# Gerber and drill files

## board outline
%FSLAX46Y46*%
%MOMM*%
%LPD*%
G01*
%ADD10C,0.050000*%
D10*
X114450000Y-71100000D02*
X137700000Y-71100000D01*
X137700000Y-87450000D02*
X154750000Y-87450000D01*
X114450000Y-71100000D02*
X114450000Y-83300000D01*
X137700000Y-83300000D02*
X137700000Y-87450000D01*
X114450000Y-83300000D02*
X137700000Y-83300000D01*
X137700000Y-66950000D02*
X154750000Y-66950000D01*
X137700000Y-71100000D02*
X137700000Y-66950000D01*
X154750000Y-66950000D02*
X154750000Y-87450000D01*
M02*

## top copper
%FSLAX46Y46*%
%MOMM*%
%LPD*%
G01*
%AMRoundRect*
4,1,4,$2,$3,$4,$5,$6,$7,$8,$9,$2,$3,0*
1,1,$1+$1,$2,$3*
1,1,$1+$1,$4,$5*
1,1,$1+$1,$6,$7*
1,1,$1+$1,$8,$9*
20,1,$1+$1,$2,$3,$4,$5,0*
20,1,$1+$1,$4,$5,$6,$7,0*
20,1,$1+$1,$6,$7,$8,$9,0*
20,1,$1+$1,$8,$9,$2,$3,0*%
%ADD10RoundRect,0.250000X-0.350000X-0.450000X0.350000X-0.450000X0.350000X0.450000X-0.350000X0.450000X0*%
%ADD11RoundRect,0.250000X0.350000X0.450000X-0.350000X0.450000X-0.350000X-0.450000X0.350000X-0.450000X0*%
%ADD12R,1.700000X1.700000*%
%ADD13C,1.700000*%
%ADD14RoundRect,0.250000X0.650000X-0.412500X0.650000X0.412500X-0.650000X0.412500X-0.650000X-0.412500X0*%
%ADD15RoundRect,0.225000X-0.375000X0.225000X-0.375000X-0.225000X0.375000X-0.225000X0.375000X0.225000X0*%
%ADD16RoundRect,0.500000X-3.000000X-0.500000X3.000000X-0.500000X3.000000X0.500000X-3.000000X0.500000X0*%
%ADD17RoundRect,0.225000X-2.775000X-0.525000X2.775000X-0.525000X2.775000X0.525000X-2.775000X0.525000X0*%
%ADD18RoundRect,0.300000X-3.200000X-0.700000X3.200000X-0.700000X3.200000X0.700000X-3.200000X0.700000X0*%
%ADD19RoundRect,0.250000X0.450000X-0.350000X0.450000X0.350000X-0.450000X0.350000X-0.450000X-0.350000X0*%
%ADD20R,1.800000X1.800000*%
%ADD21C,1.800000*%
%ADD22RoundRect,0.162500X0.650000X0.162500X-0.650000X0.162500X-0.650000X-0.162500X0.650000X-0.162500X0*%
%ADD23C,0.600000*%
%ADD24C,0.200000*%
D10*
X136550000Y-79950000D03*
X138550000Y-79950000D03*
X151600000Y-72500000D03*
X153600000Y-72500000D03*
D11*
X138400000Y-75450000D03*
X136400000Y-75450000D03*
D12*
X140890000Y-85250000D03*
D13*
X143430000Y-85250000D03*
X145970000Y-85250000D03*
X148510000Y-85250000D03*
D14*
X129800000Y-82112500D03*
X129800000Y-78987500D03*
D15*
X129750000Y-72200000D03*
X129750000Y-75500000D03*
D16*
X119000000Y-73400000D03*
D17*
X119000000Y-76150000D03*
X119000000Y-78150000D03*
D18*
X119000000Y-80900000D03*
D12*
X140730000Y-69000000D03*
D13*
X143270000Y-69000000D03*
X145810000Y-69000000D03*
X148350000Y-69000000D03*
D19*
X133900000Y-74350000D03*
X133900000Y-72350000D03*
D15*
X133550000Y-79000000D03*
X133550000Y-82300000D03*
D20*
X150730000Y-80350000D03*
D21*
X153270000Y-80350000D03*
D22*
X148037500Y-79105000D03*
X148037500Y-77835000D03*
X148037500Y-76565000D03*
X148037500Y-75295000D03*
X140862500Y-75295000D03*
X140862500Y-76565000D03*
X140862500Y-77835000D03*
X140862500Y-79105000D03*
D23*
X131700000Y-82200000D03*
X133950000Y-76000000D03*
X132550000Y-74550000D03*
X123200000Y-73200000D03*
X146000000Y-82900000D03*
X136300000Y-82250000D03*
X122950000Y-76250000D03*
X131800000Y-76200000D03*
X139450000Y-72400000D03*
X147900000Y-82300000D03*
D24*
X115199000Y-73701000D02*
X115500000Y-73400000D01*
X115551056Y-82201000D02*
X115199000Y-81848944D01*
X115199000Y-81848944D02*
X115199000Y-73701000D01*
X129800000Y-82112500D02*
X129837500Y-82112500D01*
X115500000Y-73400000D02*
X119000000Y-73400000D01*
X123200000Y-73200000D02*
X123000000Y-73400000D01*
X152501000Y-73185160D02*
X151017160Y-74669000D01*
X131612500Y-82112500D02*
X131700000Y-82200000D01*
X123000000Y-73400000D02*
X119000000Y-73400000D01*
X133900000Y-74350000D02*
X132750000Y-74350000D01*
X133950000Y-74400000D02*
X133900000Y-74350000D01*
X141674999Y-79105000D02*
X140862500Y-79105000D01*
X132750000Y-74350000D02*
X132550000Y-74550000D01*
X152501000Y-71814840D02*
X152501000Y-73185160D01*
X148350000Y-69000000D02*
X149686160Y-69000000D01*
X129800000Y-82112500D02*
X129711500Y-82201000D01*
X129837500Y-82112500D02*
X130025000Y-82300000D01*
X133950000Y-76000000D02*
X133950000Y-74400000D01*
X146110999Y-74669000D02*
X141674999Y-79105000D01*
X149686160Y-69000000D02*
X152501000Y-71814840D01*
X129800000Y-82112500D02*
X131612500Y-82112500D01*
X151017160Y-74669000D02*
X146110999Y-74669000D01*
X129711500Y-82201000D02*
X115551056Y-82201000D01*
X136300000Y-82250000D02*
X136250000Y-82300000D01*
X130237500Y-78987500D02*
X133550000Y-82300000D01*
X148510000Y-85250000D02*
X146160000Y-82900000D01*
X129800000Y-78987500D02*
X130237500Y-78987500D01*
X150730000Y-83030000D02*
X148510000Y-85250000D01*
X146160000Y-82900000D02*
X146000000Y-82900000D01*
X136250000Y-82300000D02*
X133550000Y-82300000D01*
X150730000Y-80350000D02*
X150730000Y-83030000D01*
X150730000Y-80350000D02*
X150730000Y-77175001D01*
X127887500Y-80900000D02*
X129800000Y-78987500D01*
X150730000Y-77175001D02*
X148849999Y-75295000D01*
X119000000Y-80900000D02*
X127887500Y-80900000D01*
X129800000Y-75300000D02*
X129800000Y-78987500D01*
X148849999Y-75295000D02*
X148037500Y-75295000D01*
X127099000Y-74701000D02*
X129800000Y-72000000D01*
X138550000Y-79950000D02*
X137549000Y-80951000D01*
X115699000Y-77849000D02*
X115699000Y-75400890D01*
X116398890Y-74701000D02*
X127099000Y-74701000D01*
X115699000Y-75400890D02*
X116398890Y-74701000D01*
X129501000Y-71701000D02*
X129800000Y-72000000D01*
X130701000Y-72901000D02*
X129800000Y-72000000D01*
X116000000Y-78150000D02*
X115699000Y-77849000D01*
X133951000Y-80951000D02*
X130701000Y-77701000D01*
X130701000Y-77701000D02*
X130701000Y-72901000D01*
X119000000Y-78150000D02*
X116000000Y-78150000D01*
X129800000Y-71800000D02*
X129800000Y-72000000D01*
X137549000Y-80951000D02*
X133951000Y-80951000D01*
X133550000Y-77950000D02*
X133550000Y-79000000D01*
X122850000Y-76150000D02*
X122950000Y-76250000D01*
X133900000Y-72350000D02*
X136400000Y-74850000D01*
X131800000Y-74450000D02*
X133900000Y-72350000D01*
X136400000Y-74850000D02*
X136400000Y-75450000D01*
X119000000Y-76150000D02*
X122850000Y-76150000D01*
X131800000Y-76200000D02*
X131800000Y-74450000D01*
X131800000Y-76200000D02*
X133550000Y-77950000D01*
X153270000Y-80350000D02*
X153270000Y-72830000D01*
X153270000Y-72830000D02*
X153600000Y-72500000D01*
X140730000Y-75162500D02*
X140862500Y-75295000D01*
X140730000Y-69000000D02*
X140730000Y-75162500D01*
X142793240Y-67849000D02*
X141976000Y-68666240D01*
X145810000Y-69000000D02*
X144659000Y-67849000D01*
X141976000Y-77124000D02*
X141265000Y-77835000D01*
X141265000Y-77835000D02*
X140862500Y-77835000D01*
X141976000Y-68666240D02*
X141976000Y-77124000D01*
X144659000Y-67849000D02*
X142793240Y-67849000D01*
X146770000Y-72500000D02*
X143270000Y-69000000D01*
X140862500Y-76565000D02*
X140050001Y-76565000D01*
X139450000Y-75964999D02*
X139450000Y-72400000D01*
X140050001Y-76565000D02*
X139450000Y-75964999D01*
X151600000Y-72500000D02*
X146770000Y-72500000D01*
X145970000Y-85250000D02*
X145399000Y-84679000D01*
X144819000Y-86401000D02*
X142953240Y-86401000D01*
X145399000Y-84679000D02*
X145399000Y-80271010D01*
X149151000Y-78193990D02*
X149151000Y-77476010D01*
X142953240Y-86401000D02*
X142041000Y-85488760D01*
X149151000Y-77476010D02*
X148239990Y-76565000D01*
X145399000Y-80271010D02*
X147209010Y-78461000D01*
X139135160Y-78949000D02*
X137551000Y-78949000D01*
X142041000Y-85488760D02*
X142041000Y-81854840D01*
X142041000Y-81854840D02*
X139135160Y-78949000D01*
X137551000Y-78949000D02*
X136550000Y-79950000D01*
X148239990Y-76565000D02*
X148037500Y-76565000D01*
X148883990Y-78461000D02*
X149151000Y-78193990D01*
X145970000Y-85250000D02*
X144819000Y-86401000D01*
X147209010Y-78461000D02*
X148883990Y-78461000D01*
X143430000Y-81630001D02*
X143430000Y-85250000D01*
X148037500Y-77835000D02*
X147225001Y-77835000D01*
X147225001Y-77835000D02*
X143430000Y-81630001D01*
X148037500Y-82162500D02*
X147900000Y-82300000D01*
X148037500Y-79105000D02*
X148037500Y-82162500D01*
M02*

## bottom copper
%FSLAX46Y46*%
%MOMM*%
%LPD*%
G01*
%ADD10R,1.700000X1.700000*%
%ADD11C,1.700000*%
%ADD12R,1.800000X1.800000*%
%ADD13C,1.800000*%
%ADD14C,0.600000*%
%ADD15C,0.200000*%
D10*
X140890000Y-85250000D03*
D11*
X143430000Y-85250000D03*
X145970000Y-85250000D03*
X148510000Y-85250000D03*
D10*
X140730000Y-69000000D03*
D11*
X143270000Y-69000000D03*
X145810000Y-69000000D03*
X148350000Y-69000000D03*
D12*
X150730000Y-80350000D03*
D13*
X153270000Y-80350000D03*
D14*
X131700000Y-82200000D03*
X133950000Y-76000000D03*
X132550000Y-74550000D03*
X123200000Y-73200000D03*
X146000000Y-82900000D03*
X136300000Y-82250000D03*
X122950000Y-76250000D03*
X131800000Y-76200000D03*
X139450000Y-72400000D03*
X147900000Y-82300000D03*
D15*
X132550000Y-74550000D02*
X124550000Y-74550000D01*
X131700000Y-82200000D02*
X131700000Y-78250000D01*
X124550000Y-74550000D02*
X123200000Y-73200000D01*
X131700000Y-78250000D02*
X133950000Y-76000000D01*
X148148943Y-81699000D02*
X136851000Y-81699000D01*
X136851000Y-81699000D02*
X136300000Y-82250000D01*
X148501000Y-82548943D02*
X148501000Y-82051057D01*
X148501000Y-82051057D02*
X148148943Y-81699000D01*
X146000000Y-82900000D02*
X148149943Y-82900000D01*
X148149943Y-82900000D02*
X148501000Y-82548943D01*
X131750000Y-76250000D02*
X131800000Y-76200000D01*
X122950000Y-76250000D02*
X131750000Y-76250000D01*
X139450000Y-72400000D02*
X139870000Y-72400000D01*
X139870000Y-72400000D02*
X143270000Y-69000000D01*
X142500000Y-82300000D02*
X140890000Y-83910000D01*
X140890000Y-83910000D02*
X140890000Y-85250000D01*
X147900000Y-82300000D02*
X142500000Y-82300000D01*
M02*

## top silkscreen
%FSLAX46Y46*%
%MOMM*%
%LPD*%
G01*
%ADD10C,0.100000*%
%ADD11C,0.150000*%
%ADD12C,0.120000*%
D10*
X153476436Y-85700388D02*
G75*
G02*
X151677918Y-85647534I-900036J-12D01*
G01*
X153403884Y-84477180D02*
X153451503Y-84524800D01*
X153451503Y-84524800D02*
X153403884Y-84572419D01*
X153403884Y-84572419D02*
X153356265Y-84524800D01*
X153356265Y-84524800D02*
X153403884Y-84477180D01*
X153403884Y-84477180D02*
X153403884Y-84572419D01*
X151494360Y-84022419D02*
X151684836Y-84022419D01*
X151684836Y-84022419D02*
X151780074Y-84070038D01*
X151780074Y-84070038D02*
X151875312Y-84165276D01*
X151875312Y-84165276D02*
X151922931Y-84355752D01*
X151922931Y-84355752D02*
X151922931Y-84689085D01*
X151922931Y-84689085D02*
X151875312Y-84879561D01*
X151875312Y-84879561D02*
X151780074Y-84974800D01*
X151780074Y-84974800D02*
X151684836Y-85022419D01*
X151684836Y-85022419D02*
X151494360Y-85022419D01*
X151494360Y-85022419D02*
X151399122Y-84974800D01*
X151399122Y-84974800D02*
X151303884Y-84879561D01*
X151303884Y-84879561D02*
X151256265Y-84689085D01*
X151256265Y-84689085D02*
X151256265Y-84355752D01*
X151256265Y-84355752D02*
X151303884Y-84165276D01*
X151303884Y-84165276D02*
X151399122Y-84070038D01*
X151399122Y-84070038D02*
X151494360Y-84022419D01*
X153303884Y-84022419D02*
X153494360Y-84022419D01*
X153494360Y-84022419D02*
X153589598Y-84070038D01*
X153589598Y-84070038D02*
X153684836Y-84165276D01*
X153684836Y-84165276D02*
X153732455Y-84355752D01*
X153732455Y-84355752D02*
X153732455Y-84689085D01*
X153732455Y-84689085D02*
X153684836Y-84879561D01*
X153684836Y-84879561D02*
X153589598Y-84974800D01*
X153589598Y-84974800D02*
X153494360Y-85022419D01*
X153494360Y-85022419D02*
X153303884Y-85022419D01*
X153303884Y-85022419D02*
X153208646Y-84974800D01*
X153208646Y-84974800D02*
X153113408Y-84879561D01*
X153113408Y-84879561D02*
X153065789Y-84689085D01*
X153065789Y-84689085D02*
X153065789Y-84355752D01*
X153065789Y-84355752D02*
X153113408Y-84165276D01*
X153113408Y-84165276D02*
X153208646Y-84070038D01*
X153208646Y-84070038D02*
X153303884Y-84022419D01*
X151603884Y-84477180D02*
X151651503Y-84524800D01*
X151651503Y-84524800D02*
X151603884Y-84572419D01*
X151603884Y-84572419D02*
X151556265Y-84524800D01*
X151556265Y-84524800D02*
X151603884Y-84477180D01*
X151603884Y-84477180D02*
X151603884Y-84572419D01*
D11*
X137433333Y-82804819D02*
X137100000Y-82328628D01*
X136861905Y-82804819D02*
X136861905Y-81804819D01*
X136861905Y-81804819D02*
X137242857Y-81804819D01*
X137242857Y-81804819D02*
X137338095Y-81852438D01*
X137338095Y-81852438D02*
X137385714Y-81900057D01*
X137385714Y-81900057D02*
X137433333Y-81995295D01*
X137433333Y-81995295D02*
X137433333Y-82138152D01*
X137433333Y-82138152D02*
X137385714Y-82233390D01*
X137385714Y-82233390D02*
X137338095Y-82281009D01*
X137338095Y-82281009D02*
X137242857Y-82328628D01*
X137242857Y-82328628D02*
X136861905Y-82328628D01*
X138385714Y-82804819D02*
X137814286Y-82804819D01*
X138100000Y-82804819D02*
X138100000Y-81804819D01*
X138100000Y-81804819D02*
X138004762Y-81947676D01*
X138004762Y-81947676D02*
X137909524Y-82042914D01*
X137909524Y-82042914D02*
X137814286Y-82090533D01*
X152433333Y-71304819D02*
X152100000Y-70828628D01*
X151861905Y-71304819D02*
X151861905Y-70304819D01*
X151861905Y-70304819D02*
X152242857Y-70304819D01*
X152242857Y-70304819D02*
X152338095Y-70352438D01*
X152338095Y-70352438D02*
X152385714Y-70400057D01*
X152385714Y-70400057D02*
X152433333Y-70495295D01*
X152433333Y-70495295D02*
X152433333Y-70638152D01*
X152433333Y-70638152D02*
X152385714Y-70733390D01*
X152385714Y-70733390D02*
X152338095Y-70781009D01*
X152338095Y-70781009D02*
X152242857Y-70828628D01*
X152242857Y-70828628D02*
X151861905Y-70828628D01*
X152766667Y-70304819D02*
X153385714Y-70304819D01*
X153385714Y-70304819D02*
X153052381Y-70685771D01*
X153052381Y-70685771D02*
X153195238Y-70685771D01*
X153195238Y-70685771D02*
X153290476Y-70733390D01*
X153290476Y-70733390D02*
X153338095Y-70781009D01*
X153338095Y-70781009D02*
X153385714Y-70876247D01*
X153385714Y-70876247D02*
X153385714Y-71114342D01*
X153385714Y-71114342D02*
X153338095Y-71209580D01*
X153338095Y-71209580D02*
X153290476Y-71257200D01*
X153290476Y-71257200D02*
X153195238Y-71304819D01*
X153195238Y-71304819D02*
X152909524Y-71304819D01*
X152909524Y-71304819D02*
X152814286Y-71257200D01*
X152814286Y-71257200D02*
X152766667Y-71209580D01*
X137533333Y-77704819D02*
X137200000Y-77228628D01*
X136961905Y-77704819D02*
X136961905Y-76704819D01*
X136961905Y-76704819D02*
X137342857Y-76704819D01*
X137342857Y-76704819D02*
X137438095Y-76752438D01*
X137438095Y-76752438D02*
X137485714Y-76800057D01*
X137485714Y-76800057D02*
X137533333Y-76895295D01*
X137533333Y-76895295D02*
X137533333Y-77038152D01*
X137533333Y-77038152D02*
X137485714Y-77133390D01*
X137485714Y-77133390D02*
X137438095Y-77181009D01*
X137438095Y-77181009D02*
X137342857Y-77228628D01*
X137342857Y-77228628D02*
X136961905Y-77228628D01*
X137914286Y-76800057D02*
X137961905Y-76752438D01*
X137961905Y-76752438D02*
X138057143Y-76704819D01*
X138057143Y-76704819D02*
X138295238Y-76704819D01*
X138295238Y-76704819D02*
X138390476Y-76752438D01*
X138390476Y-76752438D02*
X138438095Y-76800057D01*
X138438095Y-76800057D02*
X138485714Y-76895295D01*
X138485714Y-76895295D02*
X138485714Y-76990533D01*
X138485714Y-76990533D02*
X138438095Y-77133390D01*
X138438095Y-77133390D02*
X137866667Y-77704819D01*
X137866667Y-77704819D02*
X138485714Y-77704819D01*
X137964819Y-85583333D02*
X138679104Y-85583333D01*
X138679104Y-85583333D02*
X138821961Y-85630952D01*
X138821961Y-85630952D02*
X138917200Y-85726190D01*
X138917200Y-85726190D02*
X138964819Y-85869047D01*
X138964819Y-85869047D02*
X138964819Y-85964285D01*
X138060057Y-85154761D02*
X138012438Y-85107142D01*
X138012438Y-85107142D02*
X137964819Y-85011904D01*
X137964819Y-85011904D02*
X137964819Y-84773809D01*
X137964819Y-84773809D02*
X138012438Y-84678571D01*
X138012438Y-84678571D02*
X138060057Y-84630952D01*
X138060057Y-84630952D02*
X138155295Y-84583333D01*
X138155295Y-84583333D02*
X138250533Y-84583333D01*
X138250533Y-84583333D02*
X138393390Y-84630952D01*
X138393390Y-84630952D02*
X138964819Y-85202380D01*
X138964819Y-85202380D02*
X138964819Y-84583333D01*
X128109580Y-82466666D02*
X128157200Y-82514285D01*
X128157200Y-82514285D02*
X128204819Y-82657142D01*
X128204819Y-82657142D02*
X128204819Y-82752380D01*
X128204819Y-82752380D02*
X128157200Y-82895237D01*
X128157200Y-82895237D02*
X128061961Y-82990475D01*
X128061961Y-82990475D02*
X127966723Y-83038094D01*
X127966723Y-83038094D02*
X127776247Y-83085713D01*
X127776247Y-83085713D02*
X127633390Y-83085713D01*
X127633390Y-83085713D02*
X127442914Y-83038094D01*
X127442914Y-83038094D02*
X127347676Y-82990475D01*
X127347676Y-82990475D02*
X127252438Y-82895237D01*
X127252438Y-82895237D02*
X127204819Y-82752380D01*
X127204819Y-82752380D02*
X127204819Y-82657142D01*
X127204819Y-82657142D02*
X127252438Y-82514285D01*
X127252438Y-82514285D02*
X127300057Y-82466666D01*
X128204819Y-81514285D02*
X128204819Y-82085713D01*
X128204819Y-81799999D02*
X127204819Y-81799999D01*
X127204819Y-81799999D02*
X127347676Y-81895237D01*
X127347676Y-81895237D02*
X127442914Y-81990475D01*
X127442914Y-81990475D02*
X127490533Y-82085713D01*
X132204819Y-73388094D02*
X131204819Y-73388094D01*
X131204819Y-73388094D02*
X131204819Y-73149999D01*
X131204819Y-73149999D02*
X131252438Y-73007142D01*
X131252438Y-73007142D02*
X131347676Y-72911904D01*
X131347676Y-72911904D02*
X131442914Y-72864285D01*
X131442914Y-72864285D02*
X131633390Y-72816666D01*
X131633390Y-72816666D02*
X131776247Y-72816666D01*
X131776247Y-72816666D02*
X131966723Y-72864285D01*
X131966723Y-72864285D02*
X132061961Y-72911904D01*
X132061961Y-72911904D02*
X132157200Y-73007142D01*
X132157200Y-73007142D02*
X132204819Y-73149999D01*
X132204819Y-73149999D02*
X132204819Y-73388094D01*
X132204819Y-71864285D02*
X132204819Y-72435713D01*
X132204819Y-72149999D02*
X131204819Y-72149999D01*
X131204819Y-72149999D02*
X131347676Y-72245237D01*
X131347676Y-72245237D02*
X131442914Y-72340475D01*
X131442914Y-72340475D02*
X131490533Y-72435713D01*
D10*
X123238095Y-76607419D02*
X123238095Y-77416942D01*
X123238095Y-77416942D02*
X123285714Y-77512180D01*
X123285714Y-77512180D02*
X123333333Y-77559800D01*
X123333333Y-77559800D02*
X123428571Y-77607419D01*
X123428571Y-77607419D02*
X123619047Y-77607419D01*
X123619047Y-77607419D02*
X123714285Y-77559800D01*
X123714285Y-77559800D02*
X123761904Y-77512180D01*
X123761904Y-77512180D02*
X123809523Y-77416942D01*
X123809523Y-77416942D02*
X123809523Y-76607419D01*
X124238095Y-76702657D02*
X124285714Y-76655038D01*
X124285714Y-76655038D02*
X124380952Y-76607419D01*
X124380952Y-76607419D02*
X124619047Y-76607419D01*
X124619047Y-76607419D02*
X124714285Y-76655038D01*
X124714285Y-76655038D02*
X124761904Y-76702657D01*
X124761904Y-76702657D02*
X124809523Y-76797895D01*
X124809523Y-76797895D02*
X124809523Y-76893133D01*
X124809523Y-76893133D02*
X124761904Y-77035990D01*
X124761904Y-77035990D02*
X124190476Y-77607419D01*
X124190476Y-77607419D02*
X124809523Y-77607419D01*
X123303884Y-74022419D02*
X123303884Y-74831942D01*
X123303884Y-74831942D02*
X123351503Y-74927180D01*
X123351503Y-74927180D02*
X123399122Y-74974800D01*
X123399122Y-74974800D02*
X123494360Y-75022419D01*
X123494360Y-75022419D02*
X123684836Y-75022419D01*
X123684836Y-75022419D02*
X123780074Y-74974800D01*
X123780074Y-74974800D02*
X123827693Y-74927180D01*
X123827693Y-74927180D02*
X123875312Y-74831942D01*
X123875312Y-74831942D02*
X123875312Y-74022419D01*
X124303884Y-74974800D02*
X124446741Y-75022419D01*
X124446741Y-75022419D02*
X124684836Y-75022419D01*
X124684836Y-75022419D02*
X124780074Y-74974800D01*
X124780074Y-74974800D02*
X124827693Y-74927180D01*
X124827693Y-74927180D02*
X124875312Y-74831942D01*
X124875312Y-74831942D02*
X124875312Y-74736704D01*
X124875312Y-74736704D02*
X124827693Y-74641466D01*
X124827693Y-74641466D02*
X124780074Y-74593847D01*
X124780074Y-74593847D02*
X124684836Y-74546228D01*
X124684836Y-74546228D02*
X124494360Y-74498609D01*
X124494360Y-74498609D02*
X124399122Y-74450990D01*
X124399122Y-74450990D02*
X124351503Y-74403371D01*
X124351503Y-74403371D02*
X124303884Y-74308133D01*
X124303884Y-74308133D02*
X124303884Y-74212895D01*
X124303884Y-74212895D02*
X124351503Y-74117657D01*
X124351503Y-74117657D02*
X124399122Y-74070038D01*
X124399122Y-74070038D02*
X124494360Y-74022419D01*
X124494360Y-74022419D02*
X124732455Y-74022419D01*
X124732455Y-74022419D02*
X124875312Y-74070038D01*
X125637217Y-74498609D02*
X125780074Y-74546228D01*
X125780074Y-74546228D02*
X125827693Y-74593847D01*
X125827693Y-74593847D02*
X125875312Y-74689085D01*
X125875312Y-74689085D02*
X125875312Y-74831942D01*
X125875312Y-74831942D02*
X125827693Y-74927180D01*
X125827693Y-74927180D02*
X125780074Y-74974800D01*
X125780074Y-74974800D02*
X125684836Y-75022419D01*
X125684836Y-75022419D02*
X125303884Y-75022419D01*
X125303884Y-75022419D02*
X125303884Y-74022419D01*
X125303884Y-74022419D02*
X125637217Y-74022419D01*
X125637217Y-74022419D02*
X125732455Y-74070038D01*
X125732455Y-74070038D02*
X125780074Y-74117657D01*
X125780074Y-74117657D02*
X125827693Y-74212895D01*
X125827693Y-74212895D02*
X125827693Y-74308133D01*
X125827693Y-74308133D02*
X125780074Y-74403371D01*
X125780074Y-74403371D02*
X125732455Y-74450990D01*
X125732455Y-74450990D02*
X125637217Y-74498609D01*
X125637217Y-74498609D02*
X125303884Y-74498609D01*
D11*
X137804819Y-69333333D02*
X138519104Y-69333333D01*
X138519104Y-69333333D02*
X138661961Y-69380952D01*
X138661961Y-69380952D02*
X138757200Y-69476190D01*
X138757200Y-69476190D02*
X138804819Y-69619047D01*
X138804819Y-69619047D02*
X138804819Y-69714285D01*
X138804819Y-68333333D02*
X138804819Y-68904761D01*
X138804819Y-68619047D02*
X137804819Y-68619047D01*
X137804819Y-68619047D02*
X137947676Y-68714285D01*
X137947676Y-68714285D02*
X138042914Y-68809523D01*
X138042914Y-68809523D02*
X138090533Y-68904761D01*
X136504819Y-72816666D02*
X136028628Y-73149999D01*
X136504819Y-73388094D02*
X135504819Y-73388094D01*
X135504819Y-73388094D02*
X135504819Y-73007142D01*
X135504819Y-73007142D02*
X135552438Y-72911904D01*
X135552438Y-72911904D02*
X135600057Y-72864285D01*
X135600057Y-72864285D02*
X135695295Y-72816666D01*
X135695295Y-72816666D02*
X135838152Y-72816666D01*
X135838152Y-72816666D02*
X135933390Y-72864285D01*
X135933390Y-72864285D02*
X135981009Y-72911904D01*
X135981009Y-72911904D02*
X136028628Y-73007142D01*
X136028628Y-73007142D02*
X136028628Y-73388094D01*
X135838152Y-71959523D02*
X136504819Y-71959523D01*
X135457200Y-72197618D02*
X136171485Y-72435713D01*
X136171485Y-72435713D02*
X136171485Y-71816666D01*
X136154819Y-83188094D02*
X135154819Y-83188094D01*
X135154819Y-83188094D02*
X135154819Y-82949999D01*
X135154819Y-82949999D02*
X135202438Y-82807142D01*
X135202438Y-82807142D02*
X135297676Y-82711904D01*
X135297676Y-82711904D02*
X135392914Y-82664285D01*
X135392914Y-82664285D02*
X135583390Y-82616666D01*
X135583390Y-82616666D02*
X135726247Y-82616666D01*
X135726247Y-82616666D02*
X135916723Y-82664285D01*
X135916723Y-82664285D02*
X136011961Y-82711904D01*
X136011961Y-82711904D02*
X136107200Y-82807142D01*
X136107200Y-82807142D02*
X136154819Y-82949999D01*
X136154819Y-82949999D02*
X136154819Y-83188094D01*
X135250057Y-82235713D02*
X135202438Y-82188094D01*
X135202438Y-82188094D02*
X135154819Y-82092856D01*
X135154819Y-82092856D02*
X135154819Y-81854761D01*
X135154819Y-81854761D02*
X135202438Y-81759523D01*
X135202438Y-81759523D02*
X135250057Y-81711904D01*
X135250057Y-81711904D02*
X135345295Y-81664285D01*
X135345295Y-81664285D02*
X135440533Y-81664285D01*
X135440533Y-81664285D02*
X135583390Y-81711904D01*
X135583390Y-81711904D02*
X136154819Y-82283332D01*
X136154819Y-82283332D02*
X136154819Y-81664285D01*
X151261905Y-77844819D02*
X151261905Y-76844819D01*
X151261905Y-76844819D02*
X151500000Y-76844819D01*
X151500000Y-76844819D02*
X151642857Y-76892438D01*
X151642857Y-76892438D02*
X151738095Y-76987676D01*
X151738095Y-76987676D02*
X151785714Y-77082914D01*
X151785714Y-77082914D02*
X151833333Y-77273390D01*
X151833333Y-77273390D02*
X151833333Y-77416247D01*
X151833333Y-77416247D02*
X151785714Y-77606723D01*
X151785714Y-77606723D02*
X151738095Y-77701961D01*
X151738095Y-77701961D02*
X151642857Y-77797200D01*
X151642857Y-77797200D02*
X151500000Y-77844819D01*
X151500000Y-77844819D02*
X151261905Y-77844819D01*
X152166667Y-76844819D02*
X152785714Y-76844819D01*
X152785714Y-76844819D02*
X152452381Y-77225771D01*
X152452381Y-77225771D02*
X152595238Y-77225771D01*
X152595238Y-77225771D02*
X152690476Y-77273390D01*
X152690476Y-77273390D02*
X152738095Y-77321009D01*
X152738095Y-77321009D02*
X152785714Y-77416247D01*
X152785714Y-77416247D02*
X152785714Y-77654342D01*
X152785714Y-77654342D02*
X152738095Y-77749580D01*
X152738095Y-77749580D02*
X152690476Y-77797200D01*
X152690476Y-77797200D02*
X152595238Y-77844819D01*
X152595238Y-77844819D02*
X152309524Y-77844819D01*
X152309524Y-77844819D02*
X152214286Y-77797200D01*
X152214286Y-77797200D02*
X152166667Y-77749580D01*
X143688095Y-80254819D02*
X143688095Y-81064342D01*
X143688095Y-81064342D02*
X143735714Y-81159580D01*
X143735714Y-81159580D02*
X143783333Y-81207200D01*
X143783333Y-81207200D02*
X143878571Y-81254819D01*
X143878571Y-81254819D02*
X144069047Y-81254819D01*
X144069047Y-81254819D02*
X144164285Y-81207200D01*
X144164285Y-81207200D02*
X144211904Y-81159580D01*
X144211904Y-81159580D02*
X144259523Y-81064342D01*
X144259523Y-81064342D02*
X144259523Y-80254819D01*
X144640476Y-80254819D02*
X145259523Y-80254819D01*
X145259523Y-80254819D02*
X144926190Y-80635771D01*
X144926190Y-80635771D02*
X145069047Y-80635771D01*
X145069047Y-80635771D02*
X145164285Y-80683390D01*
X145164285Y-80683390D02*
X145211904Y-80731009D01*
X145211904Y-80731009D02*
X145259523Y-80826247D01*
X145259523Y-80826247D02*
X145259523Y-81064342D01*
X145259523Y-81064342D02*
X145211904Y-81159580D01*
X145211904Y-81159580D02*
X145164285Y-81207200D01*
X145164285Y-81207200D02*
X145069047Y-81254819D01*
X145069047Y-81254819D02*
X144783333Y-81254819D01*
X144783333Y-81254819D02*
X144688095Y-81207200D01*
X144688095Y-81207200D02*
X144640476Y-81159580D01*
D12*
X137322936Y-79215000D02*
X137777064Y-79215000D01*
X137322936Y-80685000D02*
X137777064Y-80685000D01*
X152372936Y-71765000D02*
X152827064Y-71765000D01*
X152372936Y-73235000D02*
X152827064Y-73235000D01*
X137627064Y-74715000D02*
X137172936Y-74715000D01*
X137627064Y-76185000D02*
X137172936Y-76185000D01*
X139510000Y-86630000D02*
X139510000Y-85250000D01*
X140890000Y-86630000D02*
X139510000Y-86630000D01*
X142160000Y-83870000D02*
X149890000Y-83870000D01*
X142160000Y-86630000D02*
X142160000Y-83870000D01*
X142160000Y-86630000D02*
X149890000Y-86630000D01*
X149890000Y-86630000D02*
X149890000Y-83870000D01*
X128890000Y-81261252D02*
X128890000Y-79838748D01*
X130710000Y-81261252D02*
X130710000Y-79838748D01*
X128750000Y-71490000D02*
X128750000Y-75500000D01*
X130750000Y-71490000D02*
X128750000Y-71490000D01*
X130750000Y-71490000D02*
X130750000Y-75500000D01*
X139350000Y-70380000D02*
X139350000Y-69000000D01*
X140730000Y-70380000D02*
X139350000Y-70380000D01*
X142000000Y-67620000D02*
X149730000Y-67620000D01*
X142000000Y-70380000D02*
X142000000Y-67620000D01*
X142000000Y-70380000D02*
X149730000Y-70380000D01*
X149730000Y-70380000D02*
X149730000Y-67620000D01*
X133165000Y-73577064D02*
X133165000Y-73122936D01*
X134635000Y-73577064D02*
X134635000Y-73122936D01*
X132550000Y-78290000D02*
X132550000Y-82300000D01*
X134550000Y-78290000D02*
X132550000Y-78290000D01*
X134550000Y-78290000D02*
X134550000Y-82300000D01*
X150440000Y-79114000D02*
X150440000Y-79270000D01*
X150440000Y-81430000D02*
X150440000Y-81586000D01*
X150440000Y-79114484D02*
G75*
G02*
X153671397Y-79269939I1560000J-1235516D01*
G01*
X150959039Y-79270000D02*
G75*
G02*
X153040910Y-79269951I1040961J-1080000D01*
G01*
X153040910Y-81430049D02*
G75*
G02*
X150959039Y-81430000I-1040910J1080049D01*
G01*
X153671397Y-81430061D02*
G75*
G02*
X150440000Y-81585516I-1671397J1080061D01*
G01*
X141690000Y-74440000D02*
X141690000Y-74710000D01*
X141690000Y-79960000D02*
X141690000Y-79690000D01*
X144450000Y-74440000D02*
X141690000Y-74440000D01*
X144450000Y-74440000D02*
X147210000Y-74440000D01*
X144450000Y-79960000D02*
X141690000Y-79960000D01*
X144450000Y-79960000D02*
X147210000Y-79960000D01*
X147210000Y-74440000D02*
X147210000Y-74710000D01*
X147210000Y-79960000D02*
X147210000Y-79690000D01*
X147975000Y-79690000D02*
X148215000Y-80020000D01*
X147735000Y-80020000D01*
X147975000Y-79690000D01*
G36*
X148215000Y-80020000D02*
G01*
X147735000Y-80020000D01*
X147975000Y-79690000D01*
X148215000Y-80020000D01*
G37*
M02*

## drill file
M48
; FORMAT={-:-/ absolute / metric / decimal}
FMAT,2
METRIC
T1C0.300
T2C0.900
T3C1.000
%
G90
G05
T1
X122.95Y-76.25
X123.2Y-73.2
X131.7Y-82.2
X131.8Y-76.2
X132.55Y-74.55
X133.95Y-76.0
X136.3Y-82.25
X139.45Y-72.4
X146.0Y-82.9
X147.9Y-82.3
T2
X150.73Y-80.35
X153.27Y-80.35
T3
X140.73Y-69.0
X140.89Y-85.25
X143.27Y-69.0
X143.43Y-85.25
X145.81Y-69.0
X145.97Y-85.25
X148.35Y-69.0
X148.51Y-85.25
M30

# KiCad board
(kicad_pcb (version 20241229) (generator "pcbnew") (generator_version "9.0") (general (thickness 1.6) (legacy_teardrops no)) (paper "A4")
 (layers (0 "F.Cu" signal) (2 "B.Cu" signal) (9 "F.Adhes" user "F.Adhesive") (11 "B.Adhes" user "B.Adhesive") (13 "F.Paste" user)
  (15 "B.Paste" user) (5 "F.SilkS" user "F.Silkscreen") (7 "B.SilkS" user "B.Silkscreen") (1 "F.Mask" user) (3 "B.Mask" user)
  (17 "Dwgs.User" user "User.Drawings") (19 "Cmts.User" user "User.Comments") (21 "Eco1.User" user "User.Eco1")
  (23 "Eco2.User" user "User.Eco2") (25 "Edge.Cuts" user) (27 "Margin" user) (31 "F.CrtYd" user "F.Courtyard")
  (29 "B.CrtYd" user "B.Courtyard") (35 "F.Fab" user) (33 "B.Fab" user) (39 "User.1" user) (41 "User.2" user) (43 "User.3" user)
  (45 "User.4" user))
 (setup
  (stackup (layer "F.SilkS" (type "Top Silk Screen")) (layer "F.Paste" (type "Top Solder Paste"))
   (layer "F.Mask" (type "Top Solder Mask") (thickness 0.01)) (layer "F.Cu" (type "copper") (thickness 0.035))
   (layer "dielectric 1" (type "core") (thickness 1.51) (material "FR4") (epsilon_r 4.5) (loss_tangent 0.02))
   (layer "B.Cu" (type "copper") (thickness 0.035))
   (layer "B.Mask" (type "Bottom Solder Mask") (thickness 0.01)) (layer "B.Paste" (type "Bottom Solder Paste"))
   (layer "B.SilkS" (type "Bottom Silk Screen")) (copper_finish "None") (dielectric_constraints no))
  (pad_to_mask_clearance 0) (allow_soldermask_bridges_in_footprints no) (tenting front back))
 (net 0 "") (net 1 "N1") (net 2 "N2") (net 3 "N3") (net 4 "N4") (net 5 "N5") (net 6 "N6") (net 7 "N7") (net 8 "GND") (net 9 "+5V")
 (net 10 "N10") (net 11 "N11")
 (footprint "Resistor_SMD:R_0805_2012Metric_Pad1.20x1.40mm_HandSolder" (layer "F.Cu") (at 137.55 79.95)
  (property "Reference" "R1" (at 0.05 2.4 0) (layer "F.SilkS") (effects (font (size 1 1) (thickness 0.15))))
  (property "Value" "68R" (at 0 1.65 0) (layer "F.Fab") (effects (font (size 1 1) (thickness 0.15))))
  (fp_line (start -0.227064 -0.735) (end 0.227064 -0.735) (stroke (width 0.12) (type solid)) (layer "F.SilkS"))
  (fp_line (start -0.227064 0.735) (end 0.227064 0.735) (stroke (width 0.12) (type solid)) (layer "F.SilkS"))
  (pad "1" smd roundrect (at -1 0) (size 1.2 1.4) (layers "F.Cu" "F.Mask" "F.Paste") (roundrect_rratio 0.208333) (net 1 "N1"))
  (pad "2" smd roundrect (at 1 0) (size 1.2 1.4) (layers "F.Cu" "F.Mask" "F.Paste") (roundrect_rratio 0.208333) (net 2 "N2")))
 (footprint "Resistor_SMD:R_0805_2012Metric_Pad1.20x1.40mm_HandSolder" (layer "F.Cu") (at 152.6 72.5)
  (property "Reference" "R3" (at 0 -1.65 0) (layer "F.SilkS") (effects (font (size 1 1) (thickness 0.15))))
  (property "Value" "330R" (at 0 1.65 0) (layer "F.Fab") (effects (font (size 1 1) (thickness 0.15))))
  (fp_line (start -0.227064 -0.735) (end 0.227064 -0.735) (stroke (width 0.12) (type solid)) (layer "F.SilkS"))
  (fp_line (start -0.227064 0.735) (end 0.227064 0.735) (stroke (width 0.12) (type solid)) (layer "F.SilkS"))
  (pad "1" smd roundrect (at -1 0) (size 1.2 1.4) (layers "F.Cu" "F.Mask" "F.Paste") (roundrect_rratio 0.208333) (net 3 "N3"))
  (pad "2" smd roundrect (at 1 0) (size 1.2 1.4) (layers "F.Cu" "F.Mask" "F.Paste") (roundrect_rratio 0.208333) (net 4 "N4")))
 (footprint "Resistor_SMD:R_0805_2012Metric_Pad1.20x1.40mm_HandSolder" (layer "F.Cu") (at 137.4 75.45 180)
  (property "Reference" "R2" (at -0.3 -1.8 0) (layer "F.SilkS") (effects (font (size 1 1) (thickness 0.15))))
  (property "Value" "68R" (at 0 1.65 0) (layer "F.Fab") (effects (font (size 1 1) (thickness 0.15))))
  (fp_line (start -0.227064 0.735) (end 0.227064 0.735) (stroke (width 0.12) (type solid)) (layer "F.SilkS"))
  (fp_line (start -0.227064 -0.735) (end 0.227064 -0.735) (stroke (width 0.12) (type solid)) (layer "F.SilkS"))
  (pad "1" smd roundrect (at -1 0 180) (size 1.2 1.4) (layers "F.Cu" "F.Mask" "F.Paste") (roundrect_rratio 0.208333) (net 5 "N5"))
  (pad "2" smd roundrect (at 1 0 180) (size 1.2 1.4) (layers "F.Cu" "F.Mask" "F.Paste") (roundrect_rratio 0.208333) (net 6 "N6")))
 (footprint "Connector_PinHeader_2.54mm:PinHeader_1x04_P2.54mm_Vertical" (layer "F.Cu") (at 140.89 85.25 90)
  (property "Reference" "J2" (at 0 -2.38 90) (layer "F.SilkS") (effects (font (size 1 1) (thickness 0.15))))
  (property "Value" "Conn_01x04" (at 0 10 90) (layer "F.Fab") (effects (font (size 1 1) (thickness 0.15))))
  (fp_line (start -1.38 -1.38) (end 0 -1.38) (stroke (width 0.12) (type solid)) (layer "F.SilkS"))
  (fp_line (start -1.38 0) (end -1.38 -1.38) (stroke (width 0.12) (type solid)) (layer "F.SilkS"))
  (fp_line (start 1.38 1.27) (end 1.38 9) (stroke (width 0.12) (type solid)) (layer "F.SilkS"))
  (fp_line (start -1.38 1.27) (end 1.38 1.27) (stroke (width 0.12) (type solid)) (layer "F.SilkS"))
  (fp_line (start -1.38 1.27) (end -1.38 9) (stroke (width 0.12) (type solid)) (layer "F.SilkS"))
  (fp_line (start -1.38 9) (end 1.38 9) (stroke (width 0.12) (type solid)) (layer "F.SilkS"))
  (pad "1" thru_hole rect (at 0 0 90) (size 1.7 1.7) (drill 1) (layers "*.Cu" "*.Mask") (remove_unused_layers no) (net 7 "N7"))
  (pad "2" thru_hole circle (at 0 2.54 90) (size 1.7 1.7) (drill 1) (layers "*.Cu" "*.Mask") (remove_unused_layers no) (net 5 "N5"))
  (pad "3" thru_hole circle (at 0 5.08 90) (size 1.7 1.7) (drill 1) (layers "*.Cu" "*.Mask") (remove_unused_layers no) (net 1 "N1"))
  (pad "4" thru_hole circle (at 0 7.62 90) (size 1.7 1.7) (drill 1) (layers "*.Cu" "*.Mask") (remove_unused_layers no) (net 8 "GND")))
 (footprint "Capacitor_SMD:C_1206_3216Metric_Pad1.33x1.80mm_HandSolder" (layer "F.Cu") (at 129.8 80.55 90)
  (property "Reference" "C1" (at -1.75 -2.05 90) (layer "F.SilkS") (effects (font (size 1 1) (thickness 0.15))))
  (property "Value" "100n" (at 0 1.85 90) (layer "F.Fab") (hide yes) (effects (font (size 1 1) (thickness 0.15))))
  (fp_line (start -0.711252 -0.91) (end 0.711252 -0.91) (stroke (width 0.12) (type solid)) (layer "F.SilkS"))
  (fp_line (start -0.711252 0.91) (end 0.711252 0.91) (stroke (width 0.12) (type solid)) (layer "F.SilkS"))
  (pad "1" smd roundrect (at -1.5625 0 90) (size 1.325 1.8) (layers "F.Cu" "F.Mask" "F.Paste") (roundrect_rratio 0.188679) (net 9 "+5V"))
  (pad "2" smd roundrect (at 1.5625 0 90) (size 1.325 1.8) (layers "F.Cu" "F.Mask" "F.Paste") (roundrect_rratio 0.188679) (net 8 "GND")))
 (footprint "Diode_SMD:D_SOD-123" (layer "F.Cu") (at 129.75 73.85 -90)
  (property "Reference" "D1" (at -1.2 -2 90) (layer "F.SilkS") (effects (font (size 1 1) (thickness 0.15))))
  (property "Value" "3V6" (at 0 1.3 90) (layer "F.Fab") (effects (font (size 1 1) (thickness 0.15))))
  (fp_line (start -2.36 1) (end 1.65 1) (stroke (width 0.12) (type solid)) (layer "F.SilkS"))
  (fp_line (start -2.36 -1) (end -2.36 1) (stroke (width 0.12) (type solid)) (layer "F.SilkS"))
  (fp_line (start -2.36 -1) (end 1.65 -1) (stroke (width 0.12) (type solid)) (layer "F.SilkS"))
  (pad "1" smd roundrect (at -1.65 0 270) (size 0.9 1.2) (layers "F.Cu" "F.Mask" "F.Paste") (roundrect_rratio 0.25) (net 2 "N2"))
  (pad "2" smd roundrect (at 1.65 0 270) (size 0.9 1.2) (layers "F.Cu" "F.Mask" "F.Paste") (roundrect_rratio 0.25) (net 8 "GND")))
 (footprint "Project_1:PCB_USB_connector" (layer "F.Cu") (at 119 77.15)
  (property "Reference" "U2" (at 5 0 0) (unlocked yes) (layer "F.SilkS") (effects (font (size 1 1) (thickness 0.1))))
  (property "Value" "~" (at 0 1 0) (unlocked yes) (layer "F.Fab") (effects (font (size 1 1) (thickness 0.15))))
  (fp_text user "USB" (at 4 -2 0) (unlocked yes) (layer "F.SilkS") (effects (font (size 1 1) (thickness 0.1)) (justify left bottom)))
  (pad "1" smd roundrect (at 0 -3.75) (size 7 2) (layers "F.Cu" "F.Mask" "F.Paste") (roundrect_rratio 0.25) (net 9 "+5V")
   (thermal_bridge_angle 45))
  (pad "2" smd roundrect (at 0 -1) (size 6 1.5) (layers "F.Cu" "F.Mask" "F.Paste") (roundrect_rratio 0.15) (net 6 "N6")
   (thermal_bridge_angle 45))
  (pad "3" smd roundrect (at 0 1) (size 6 1.5) (layers "F.Cu" "F.Mask" "F.Paste") (roundrect_rratio 0.15) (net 2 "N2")
   (thermal_bridge_angle 45))
  (pad "4" smd roundrect (at 0 3.75) (size 7 2) (layers "F.Cu" "F.Mask" "F.Paste") (roundrect_rratio 0.15) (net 8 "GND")
   (thermal_bridge_angle 45)))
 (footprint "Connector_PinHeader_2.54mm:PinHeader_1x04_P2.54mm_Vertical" (layer "F.Cu") (at 140.73 69 90)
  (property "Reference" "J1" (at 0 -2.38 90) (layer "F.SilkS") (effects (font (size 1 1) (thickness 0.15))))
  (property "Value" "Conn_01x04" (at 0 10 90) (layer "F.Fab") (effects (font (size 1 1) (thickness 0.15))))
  (fp_line (start -1.38 -1.38) (end 0 -1.38) (stroke (width 0.12) (type solid)) (layer "F.SilkS"))
  (fp_line (start -1.38 0) (end -1.38 -1.38) (stroke (width 0.12) (type solid)) (layer "F.SilkS"))
  (fp_line (start 1.38 1.27) (end 1.38 9) (stroke (width 0.12) (type solid)) (layer "F.SilkS"))
  (fp_line (start -1.38 1.27) (end 1.38 1.27) (stroke (width 0.12) (type solid)) (layer "F.SilkS"))
  (fp_line (start -1.38 1.27) (end -1.38 9) (stroke (width 0.12) (type solid)) (layer "F.SilkS"))
  (fp_line (start -1.38 9) (end 1.38 9) (stroke (width 0.12) (type solid)) (layer "F.SilkS"))
  (pad "1" thru_hole rect (at 0 0 90) (size 1.7 1.7) (drill 1) (layers "*.Cu" "*.Mask") (remove_unused_layers no) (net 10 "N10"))
  (pad "2" thru_hole circle (at 0 2.54 90) (size 1.7 1.7) (drill 1) (layers "*.Cu" "*.Mask") (remove_unused_layers no) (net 3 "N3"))
  (pad "3" thru_hole circle (at 0 5.08 90) (size 1.7 1.7) (drill 1) (layers "*.Cu" "*.Mask") (remove_unused_layers no) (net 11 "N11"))
  (pad "4" thru_hole circle (at 0 7.62 90) (size 1.7 1.7) (drill 1) (layers "*.Cu" "*.Mask") (remove_unused_layers no) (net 9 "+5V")))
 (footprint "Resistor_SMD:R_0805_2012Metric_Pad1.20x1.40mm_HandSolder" (layer "F.Cu") (at 133.9 73.35 90)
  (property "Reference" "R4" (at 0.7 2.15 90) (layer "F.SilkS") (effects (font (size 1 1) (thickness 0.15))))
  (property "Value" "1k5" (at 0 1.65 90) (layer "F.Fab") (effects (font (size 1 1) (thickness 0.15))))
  (fp_line (start -0.227064 -0.735) (end 0.227064 -0.735) (stroke (width 0.12) (type solid)) (layer "F.SilkS"))
  (fp_line (start -0.227064 0.735) (end 0.227064 0.735) (stroke (width 0.12) (type solid)) (layer "F.SilkS"))
  (pad "1" smd roundrect (at -1 0 90) (size 1.2 1.4) (layers "F.Cu" "F.Mask" "F.Paste") (roundrect_rratio 0.208333) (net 9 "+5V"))
  (pad "2" smd roundrect (at 1 0 90) (size 1.2 1.4) (layers "F.Cu" "F.Mask" "F.Paste") (roundrect_rratio 0.208333) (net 6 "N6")))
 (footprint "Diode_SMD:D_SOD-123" (layer "F.Cu") (at 133.55 80.65 -90)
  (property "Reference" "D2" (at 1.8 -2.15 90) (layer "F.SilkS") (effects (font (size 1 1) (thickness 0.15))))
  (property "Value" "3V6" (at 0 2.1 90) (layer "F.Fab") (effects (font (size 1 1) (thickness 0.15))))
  (fp_line (start -2.36 1) (end 1.65 1) (stroke (width 0.12) (type solid)) (layer "F.SilkS"))
  (fp_line (start -2.36 -1) (end -2.36 1) (stroke (width 0.12) (type solid)) (layer "F.SilkS"))
  (fp_line (start -2.36 -1) (end 1.65 -1) (stroke (width 0.12) (type solid)) (layer "F.SilkS"))
  (pad "1" smd roundrect (at -1.65 0 270) (size 0.9 1.2) (layers "F.Cu" "F.Mask" "F.Paste") (roundrect_rratio 0.25) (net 6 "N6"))
  (pad "2" smd roundrect (at 1.65 0 270) (size 0.9 1.2) (layers "F.Cu" "F.Mask" "F.Paste") (roundrect_rratio 0.25) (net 8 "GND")))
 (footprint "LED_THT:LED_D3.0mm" (layer "F.Cu") (at 150.73 80.35)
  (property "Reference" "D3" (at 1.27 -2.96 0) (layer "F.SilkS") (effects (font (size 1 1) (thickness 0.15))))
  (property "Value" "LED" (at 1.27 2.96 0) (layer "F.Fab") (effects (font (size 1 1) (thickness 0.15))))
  (fp_line (start -0.29 -1.236) (end -0.29 -1.08) (stroke (width 0.12) (type solid)) (layer "F.SilkS"))
  (fp_line (start -0.29 1.08) (end -0.29 1.236) (stroke (width 0.12) (type solid)) (layer "F.SilkS"))
  (fp_arc (start -0.29 -1.235516) (mid 1.365624 -1.987701) (end 2.941397 -1.080061) (stroke (width 0.12) (type solid)) (layer "F.SilkS"))
  (fp_arc (start 0.229039 -1.08) (mid 1.269964 -1.5) (end 2.31091 -1.080049) (stroke (width 0.12) (type solid)) (layer "F.SilkS"))
  (fp_arc (start 2.31091 1.080049) (mid 1.269964 1.5) (end 0.229039 1.08) (stroke (width 0.12) (type solid)) (layer "F.SilkS"))
  (fp_arc (start 2.941397 1.080061) (mid 1.365624 1.987701) (end -0.29 1.235516) (stroke (width 0.12) (type solid)) (layer "F.SilkS"))
  (pad "1" thru_hole rect (at 0 0) (size 1.8 1.8) (drill 0.9) (layers "*.Cu" "*.Mask") (remove_unused_layers no) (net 8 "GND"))
  (pad "2" thru_hole circle (at 2.54 0) (size 1.8 1.8) (drill 0.9) (layers "*.Cu" "*.Mask") (remove_unused_layers no) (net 4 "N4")))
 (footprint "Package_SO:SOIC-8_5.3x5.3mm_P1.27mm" (layer "F.Cu") (at 144.45 77.2 180)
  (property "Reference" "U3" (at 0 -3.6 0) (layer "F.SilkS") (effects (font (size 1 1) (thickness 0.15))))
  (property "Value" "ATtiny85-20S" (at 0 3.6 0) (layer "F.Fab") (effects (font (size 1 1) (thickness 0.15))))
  (fp_line (start 2.76 2.76) (end 2.76 2.49) (stroke (width 0.12) (type solid)) (layer "F.SilkS"))
  (fp_line (start 2.76 -2.76) (end 2.76 -2.49) (stroke (width 0.12) (type solid)) (layer "F.SilkS"))
  (fp_line (start 0 2.76) (end 2.76 2.76) (stroke (width 0.12) (type solid)) (layer "F.SilkS"))
  (fp_line (start 0 2.76) (end -2.76 2.76) (stroke (width 0.12) (type solid)) (layer "F.SilkS"))
  (fp_line (start 0 -2.76) (end 2.76 -2.76) (stroke (width 0.12) (type solid)) (layer "F.SilkS"))
  (fp_line (start 0 -2.76) (end -2.76 -2.76) (stroke (width 0.12) (type solid)) (layer "F.SilkS"))
  (fp_line (start -2.76 2.76) (end -2.76 2.49) (stroke (width 0.12) (type solid)) (layer "F.SilkS"))
  (fp_line (start -2.76 -2.76) (end -2.76 -2.49) (stroke (width 0.12) (type solid)) (layer "F.SilkS"))
  (fp_poly (pts (xy -3.525 -2.49) (xy -3.765 -2.82) (xy -3.285 -2.82)) (stroke (width 0.12) (type solid)) (fill yes) (layer "F.SilkS"))
  (pad "1" smd roundrect (at -3.5875 -1.905 180) (size 1.625 0.65) (layers "F.Cu" "F.Mask" "F.Paste") (roundrect_rratio 0.25) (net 7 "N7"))
  (pad "2" smd roundrect (at -3.5875 -0.635 180) (size 1.625 0.65) (layers "F.Cu" "F.Mask" "F.Paste") (roundrect_rratio 0.25) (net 5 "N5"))
  (pad "3" smd roundrect (at -3.5875 0.635 180) (size 1.625 0.65) (layers "F.Cu" "F.Mask" "F.Paste") (roundrect_rratio 0.25) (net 1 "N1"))
  (pad "4" smd roundrect (at -3.5875 1.905 180) (size 1.625 0.65) (layers "F.Cu" "F.Mask" "F.Paste") (roundrect_rratio 0.25) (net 8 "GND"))
  (pad "5" smd roundrect (at 3.5875 1.905 180) (size 1.625 0.65) (layers "F.Cu" "F.Mask" "F.Paste") (roundrect_rratio 0.25) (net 10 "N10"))
  (pad "6" smd roundrect (at 3.5875 0.635 180) (size 1.625 0.65) (layers "F.Cu" "F.Mask" "F.Paste") (roundrect_rratio 0.25) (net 3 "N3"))
  (pad "7" smd roundrect (at 3.5875 -0.635 180) (size 1.625 0.65) (layers "F.Cu" "F.Mask" "F.Paste") (roundrect_rratio 0.25) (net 11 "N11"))
  (pad "8" smd roundrect (at 3.5875 -1.905 180) (size 1.625 0.65) (layers "F.Cu" "F.Mask" "F.Paste") (roundrect_rratio 0.25) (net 9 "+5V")))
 (gr_arc (start 153.476436 85.700388) (mid 152.55 86.6) (end 151.677989 85.647538) (stroke (width 0.1) (type default)) (layer "F.SilkS"))
 (gr_line (start 114.45 71.1) (end 137.7 71.1) (stroke (width 0.05) (type default)) (layer "Edge.Cuts"))
 (gr_line (start 137.7 87.45) (end 154.75 87.45) (stroke (width 0.05) (type solid)) (layer "Edge.Cuts"))
 (gr_line (start 114.45 71.1) (end 114.45 83.3) (stroke (width 0.05) (type solid)) (layer "Edge.Cuts"))
 (gr_line (start 137.7 83.3) (end 137.7 87.45) (stroke (width 0.05) (type default)) (layer "Edge.Cuts"))
 (gr_line (start 114.45 83.3) (end 137.7 83.3) (stroke (width 0.05) (type default)) (layer "Edge.Cuts"))
 (gr_line (start 137.7 66.95) (end 154.75 66.95) (stroke (width 0.05) (type default)) (layer "Edge.Cuts"))
 (gr_line (start 137.7 71.1) (end 137.7 66.95) (stroke (width 0.05) (type default)) (layer "Edge.Cuts"))
 (gr_line (start 154.75 66.95) (end 154.75 87.45) (stroke (width 0.05) (type default)) (layer "Edge.Cuts"))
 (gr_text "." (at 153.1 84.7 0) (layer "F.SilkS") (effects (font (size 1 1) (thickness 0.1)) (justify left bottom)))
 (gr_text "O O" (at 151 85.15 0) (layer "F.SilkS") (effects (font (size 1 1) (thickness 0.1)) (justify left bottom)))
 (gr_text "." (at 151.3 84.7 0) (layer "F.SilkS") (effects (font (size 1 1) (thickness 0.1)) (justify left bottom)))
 (segment (start 115.199 73.701) (end 115.5 73.4) (width 0.2) (layer "F.Cu") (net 9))
 (segment (start 115.551056 82.201) (end 115.199 81.848944) (width 0.2) (layer "F.Cu") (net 9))
 (segment (start 115.199 81.848944) (end 115.199 73.701) (width 0.2) (layer "F.Cu") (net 9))
 (segment (start 129.8 82.1125) (end 129.8375 82.1125) (width 0.2) (layer "F.Cu") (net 9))
 (segment (start 115.5 73.4) (end 119 73.4) (width 0.2) (layer "F.Cu") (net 9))
 (segment (start 123.2 73.2) (end 123 73.4) (width 0.2) (layer "F.Cu") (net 9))
 (segment (start 152.501 73.18516) (end 151.01716 74.669) (width 0.2) (layer "F.Cu") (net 9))
 (segment (start 131.6125 82.1125) (end 131.7 82.2) (width 0.2) (layer "F.Cu") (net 9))
 (segment (start 123 73.4) (end 119 73.4) (width 0.2) (layer "F.Cu") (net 9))
 (segment (start 133.9 74.35) (end 132.75 74.35) (width 0.2) (layer "F.Cu") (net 9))
 (segment (start 133.95 74.4) (end 133.9 74.35) (width 0.2) (layer "F.Cu") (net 9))
 (segment (start 141.674999 79.105) (end 140.8625 79.105) (width 0.2) (layer "F.Cu") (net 9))
 (segment (start 132.75 74.35) (end 132.55 74.55) (width 0.2) (layer "F.Cu") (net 9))
 (segment (start 152.501 71.81484) (end 152.501 73.18516) (width 0.2) (layer "F.Cu") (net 9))
 (segment (start 148.35 69) (end 149.68616 69) (width 0.2) (layer "F.Cu") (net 9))
 (segment (start 129.8 82.1125) (end 129.7115 82.201) (width 0.2) (layer "F.Cu") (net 9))
 (segment (start 129.8375 82.1125) (end 130.025 82.3) (width 0.2) (layer "F.Cu") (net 9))
 (segment (start 133.95 76) (end 133.95 74.4) (width 0.2) (layer "F.Cu") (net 9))
 (segment (start 146.110999 74.669) (end 141.674999 79.105) (width 0.2) (layer "F.Cu") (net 9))
 (segment (start 149.68616 69) (end 152.501 71.81484) (width 0.2) (layer "F.Cu") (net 9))
 (segment (start 129.8 82.1125) (end 131.6125 82.1125) (width 0.2) (layer "F.Cu") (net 9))
 (segment (start 151.01716 74.669) (end 146.110999 74.669) (width 0.2) (layer "F.Cu") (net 9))
 (segment (start 129.7115 82.201) (end 115.551056 82.201) (width 0.2) (layer "F.Cu") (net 9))
 (via (at 131.7 82.2) (size 0.6) (drill 0.3) (layers "F.Cu" "B.Cu") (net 9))
 (via (at 133.95 76) (size 0.6) (drill 0.3) (layers "F.Cu" "B.Cu") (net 9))
 (via (at 132.55 74.55) (size 0.6) (drill 0.3) (layers "F.Cu" "B.Cu") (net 9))
 (via (at 123.2 73.2) (size 0.6) (drill 0.3) (layers "F.Cu" "B.Cu") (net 9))
 (segment (start 132.55 74.55) (end 124.55 74.55) (width 0.2) (layer "B.Cu") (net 9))
 (segment (start 131.7 82.2) (end 131.7 78.25) (width 0.2) (layer "B.Cu") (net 9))
 (segment (start 124.55 74.55) (end 123.2 73.2) (width 0.2) (layer "B.Cu") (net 9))
 (segment (start 131.7 78.25) (end 133.95 76) (width 0.2) (layer "B.Cu") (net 9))
 (segment (start 136.3 82.25) (end 136.25 82.3) (width 0.2) (layer "F.Cu") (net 8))
 (segment (start 130.2375 78.9875) (end 133.55 82.3) (width 0.2) (layer "F.Cu") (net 8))
 (segment (start 148.51 85.25) (end 146.16 82.9) (width 0.2) (layer "F.Cu") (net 8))
 (segment (start 129.8 78.9875) (end 130.2375 78.9875) (width 0.2) (layer "F.Cu") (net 8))
 (segment (start 150.73 83.03) (end 148.51 85.25) (width 0.2) (layer "F.Cu") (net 8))
 (segment (start 146.16 82.9) (end 146 82.9) (width 0.2) (layer "F.Cu") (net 8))
 (segment (start 136.25 82.3) (end 133.55 82.3) (width 0.2) (layer "F.Cu") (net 8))
 (segment (start 150.73 80.35) (end 150.73 83.03) (width 0.2) (layer "F.Cu") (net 8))
 (segment (start 150.73 80.35) (end 150.73 77.175001) (width 0.2) (layer "F.Cu") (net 8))
 (segment (start 127.8875 80.9) (end 129.8 78.9875) (width 0.2) (layer "F.Cu") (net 8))
 (segment (start 150.73 77.175001) (end 148.849999 75.295) (width 0.2) (layer "F.Cu") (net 8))
 (segment (start 119 80.9) (end 127.8875 80.9) (width 0.2) (layer "F.Cu") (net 8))
 (segment (start 129.8 75.3) (end 129.8 78.9875) (width 0.2) (layer "F.Cu") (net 8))
 (segment (start 148.849999 75.295) (end 148.0375 75.295) (width 0.2) (layer "F.Cu") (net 8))
 (via (at 146 82.9) (size 0.6) (drill 0.3) (layers "F.Cu" "B.Cu") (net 8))
 (via (at 136.3 82.25) (size 0.6) (drill 0.3) (layers "F.Cu" "B.Cu") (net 8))
 (segment (start 148.148943 81.699) (end 136.851 81.699) (width 0.2) (layer "B.Cu") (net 8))
 (segment (start 136.851 81.699) (end 136.3 82.25) (width 0.2) (layer "B.Cu") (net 8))
 (segment (start 148.501 82.548943) (end 148.501 82.051057) (width 0.2) (layer "B.Cu") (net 8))
 (segment (start 148.501 82.051057) (end 148.148943 81.699) (width 0.2) (layer "B.Cu") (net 8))
 (segment (start 146 82.9) (end 148.149943 82.9) (width 0.2) (layer "B.Cu") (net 8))
 (segment (start 148.149943 82.9) (end 148.501 82.548943) (width 0.2) (layer "B.Cu") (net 8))
 (segment (start 127.099 74.701) (end 129.8 72) (width 0.2) (layer "F.Cu") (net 2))
 (segment (start 138.55 79.95) (end 137.549 80.951) (width 0.2) (layer "F.Cu") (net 2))
 (segment (start 115.699 77.849) (end 115.699 75.40089) (width 0.2) (layer "F.Cu") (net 2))
 (segment (start 116.39889 74.701) (end 127.099 74.701) (width 0.2) (layer "F.Cu") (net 2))
 (segment (start 115.699 75.40089) (end 116.39889 74.701) (width 0.2) (layer "F.Cu") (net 2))
 (segment (start 129.501 71.701) (end 129.8 72) (width 0.2) (layer "F.Cu") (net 2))
 (segment (start 130.701 72.901) (end 129.8 72) (width 0.2) (layer "F.Cu") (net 2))
 (segment (start 116 78.15) (end 115.699 77.849) (width 0.2) (layer "F.Cu") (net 2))
 (segment (start 133.951 80.951) (end 130.701 77.701) (width 0.2) (layer "F.Cu") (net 2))
 (segment (start 130.701 77.701) (end 130.701 72.901) (width 0.2) (layer "F.Cu") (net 2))
 (segment (start 119 78.15) (end 116 78.15) (width 0.2) (layer "F.Cu") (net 2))
 (segment (start 129.8 71.8) (end 129.8 72) (width 0.2) (layer "F.Cu") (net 2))
 (segment (start 137.549 80.951) (end 133.951 80.951) (width 0.2) (layer "F.Cu") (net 2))
 (segment (start 133.55 77.95) (end 133.55 79) (width 0.2) (layer "F.Cu") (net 6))
 (segment (start 122.85 76.15) (end 122.95 76.25) (width 0.2) (layer "F.Cu") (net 6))
 (segment (start 133.9 72.35) (end 136.4 74.85) (width 0.2) (layer "F.Cu") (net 6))
 (segment (start 131.8 74.45) (end 133.9 72.35) (width 0.2) (layer "F.Cu") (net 6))
 (segment (start 136.4 74.85) (end 136.4 75.45) (width 0.2) (layer "F.Cu") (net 6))
 (segment (start 119 76.15) (end 122.85 76.15) (width 0.2) (layer "F.Cu") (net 6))
 (segment (start 131.8 76.2) (end 131.8 74.45) (width 0.2) (layer "F.Cu") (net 6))
 (segment (start 131.8 76.2) (end 133.55 77.95) (width 0.2) (layer "F.Cu") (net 6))
 (via (at 122.95 76.25) (size 0.6) (drill 0.3) (layers "F.Cu" "B.Cu") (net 6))
 (via (at 131.8 76.2) (size 0.6) (drill 0.3) (layers "F.Cu" "B.Cu") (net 6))
 (segment (start 131.75 76.25) (end 131.8 76.2) (width 0.2) (layer "B.Cu") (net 6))
 (segment (start 122.95 76.25) (end 131.75 76.25) (width 0.2) (layer "B.Cu") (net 6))
 (segment (start 153.27 80.35) (end 153.27 72.83) (width 0.2) (layer "F.Cu") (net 4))
 (segment (start 153.27 72.83) (end 153.6 72.5) (width 0.2) (layer "F.Cu") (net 4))
 (segment (start 140.73 75.1625) (end 140.8625 75.295) (width 0.2) (layer "F.Cu") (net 10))
 (segment (start 140.73 69) (end 140.73 75.1625) (width 0.2) (layer "F.Cu") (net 10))
 (segment (start 142.79324 67.849) (end 141.976 68.66624) (width 0.2) (layer "F.Cu") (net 11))
 (segment (start 145.81 69) (end 144.659 67.849) (width 0.2) (layer "F.Cu") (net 11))
 (segment (start 141.976 77.124) (end 141.265 77.835) (width 0.2) (layer "F.Cu") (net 11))
 (segment (start 141.265 77.835) (end 140.8625 77.835) (width 0.2) (layer "F.Cu") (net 11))
 (segment (start 141.976 68.66624) (end 141.976 77.124) (width 0.2) (layer "F.Cu") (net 11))
 (segment (start 144.659 67.849) (end 142.79324 67.849) (width 0.2) (layer "F.Cu") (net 11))
 (segment (start 146.77 72.5) (end 143.27 69) (width 0.2) (layer "F.Cu") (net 3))
 (segment (start 140.8625 76.565) (end 140.050001 76.565) (width 0.2) (layer "F.Cu") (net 3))
 (segment (start 139.45 75.964999) (end 139.45 72.4) (width 0.2) (layer "F.Cu") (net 3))
 (segment (start 140.050001 76.565) (end 139.45 75.964999) (width 0.2) (layer "F.Cu") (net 3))
 (segment (start 151.6 72.5) (end 146.77 72.5) (width 0.2) (layer "F.Cu") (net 3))
 (via (at 139.45 72.4) (size 0.6) (drill 0.3) (layers "F.Cu" "B.Cu") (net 3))
 (segment (start 139.45 72.4) (end 139.87 72.4) (width 0.2) (layer "B.Cu") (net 3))
 (segment (start 139.87 72.4) (end 143.27 69) (width 0.2) (layer "B.Cu") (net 3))
 (segment (start 145.97 85.25) (end 145.399 84.679) (width 0.2) (layer "F.Cu") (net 1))
 (segment (start 144.819 86.401) (end 142.95324 86.401) (width 0.2) (layer "F.Cu") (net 1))
 (segment (start 145.399 84.679) (end 145.399 80.27101) (width 0.2) (layer "F.Cu") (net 1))
 (segment (start 149.151 78.19399) (end 149.151 77.47601) (width 0.2) (layer "F.Cu") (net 1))
 (segment (start 142.95324 86.401) (end 142.041 85.48876) (width 0.2) (layer "F.Cu") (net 1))
 (segment (start 149.151 77.47601) (end 148.23999 76.565) (width 0.2) (layer "F.Cu") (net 1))
 (segment (start 145.399 80.27101) (end 147.20901 78.461) (width 0.2) (layer "F.Cu") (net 1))
 (segment (start 139.13516 78.949) (end 137.551 78.949) (width 0.2) (layer "F.Cu") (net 1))
 (segment (start 142.041 85.48876) (end 142.041 81.85484) (width 0.2) (layer "F.Cu") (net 1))
 (segment (start 142.041 81.85484) (end 139.13516 78.949) (width 0.2) (layer "F.Cu") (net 1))
 (segment (start 137.551 78.949) (end 136.55 79.95) (width 0.2) (layer "F.Cu") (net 1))
 (segment (start 148.23999 76.565) (end 148.0375 76.565) (width 0.2) (layer "F.Cu") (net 1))
 (segment (start 148.88399 78.461) (end 149.151 78.19399) (width 0.2) (layer "F.Cu") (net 1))
 (segment (start 145.97 85.25) (end 144.819 86.401) (width 0.2) (layer "F.Cu") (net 1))
 (segment (start 147.20901 78.461) (end 148.88399 78.461) (width 0.2) (layer "F.Cu") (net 1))
 (segment (start 143.43 81.630001) (end 143.43 85.25) (width 0.2) (layer "F.Cu") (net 5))
 (segment (start 148.0375 77.835) (end 147.225001 77.835) (width 0.2) (layer "F.Cu") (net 5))
 (segment (start 147.225001 77.835) (end 143.43 81.630001) (width 0.2) (layer "F.Cu") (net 5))
 (segment (start 148.0375 82.1625) (end 147.9 82.3) (width 0.2) (layer "F.Cu") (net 7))
 (segment (start 148.0375 79.105) (end 148.0375 82.1625) (width 0.2) (layer "F.Cu") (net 7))
 (via (at 147.9 82.3) (size 0.6) (drill 0.3) (layers "F.Cu" "B.Cu") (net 7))
 (segment (start 142.5 82.3) (end 140.89 83.91) (width 0.2) (layer "B.Cu") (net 7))
 (segment (start 140.89 83.91) (end 140.89 85.25) (width 0.2) (layer "B.Cu") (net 7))
 (segment (start 147.9 82.3) (end 142.5 82.3) (width 0.2) (layer "B.Cu") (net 7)))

